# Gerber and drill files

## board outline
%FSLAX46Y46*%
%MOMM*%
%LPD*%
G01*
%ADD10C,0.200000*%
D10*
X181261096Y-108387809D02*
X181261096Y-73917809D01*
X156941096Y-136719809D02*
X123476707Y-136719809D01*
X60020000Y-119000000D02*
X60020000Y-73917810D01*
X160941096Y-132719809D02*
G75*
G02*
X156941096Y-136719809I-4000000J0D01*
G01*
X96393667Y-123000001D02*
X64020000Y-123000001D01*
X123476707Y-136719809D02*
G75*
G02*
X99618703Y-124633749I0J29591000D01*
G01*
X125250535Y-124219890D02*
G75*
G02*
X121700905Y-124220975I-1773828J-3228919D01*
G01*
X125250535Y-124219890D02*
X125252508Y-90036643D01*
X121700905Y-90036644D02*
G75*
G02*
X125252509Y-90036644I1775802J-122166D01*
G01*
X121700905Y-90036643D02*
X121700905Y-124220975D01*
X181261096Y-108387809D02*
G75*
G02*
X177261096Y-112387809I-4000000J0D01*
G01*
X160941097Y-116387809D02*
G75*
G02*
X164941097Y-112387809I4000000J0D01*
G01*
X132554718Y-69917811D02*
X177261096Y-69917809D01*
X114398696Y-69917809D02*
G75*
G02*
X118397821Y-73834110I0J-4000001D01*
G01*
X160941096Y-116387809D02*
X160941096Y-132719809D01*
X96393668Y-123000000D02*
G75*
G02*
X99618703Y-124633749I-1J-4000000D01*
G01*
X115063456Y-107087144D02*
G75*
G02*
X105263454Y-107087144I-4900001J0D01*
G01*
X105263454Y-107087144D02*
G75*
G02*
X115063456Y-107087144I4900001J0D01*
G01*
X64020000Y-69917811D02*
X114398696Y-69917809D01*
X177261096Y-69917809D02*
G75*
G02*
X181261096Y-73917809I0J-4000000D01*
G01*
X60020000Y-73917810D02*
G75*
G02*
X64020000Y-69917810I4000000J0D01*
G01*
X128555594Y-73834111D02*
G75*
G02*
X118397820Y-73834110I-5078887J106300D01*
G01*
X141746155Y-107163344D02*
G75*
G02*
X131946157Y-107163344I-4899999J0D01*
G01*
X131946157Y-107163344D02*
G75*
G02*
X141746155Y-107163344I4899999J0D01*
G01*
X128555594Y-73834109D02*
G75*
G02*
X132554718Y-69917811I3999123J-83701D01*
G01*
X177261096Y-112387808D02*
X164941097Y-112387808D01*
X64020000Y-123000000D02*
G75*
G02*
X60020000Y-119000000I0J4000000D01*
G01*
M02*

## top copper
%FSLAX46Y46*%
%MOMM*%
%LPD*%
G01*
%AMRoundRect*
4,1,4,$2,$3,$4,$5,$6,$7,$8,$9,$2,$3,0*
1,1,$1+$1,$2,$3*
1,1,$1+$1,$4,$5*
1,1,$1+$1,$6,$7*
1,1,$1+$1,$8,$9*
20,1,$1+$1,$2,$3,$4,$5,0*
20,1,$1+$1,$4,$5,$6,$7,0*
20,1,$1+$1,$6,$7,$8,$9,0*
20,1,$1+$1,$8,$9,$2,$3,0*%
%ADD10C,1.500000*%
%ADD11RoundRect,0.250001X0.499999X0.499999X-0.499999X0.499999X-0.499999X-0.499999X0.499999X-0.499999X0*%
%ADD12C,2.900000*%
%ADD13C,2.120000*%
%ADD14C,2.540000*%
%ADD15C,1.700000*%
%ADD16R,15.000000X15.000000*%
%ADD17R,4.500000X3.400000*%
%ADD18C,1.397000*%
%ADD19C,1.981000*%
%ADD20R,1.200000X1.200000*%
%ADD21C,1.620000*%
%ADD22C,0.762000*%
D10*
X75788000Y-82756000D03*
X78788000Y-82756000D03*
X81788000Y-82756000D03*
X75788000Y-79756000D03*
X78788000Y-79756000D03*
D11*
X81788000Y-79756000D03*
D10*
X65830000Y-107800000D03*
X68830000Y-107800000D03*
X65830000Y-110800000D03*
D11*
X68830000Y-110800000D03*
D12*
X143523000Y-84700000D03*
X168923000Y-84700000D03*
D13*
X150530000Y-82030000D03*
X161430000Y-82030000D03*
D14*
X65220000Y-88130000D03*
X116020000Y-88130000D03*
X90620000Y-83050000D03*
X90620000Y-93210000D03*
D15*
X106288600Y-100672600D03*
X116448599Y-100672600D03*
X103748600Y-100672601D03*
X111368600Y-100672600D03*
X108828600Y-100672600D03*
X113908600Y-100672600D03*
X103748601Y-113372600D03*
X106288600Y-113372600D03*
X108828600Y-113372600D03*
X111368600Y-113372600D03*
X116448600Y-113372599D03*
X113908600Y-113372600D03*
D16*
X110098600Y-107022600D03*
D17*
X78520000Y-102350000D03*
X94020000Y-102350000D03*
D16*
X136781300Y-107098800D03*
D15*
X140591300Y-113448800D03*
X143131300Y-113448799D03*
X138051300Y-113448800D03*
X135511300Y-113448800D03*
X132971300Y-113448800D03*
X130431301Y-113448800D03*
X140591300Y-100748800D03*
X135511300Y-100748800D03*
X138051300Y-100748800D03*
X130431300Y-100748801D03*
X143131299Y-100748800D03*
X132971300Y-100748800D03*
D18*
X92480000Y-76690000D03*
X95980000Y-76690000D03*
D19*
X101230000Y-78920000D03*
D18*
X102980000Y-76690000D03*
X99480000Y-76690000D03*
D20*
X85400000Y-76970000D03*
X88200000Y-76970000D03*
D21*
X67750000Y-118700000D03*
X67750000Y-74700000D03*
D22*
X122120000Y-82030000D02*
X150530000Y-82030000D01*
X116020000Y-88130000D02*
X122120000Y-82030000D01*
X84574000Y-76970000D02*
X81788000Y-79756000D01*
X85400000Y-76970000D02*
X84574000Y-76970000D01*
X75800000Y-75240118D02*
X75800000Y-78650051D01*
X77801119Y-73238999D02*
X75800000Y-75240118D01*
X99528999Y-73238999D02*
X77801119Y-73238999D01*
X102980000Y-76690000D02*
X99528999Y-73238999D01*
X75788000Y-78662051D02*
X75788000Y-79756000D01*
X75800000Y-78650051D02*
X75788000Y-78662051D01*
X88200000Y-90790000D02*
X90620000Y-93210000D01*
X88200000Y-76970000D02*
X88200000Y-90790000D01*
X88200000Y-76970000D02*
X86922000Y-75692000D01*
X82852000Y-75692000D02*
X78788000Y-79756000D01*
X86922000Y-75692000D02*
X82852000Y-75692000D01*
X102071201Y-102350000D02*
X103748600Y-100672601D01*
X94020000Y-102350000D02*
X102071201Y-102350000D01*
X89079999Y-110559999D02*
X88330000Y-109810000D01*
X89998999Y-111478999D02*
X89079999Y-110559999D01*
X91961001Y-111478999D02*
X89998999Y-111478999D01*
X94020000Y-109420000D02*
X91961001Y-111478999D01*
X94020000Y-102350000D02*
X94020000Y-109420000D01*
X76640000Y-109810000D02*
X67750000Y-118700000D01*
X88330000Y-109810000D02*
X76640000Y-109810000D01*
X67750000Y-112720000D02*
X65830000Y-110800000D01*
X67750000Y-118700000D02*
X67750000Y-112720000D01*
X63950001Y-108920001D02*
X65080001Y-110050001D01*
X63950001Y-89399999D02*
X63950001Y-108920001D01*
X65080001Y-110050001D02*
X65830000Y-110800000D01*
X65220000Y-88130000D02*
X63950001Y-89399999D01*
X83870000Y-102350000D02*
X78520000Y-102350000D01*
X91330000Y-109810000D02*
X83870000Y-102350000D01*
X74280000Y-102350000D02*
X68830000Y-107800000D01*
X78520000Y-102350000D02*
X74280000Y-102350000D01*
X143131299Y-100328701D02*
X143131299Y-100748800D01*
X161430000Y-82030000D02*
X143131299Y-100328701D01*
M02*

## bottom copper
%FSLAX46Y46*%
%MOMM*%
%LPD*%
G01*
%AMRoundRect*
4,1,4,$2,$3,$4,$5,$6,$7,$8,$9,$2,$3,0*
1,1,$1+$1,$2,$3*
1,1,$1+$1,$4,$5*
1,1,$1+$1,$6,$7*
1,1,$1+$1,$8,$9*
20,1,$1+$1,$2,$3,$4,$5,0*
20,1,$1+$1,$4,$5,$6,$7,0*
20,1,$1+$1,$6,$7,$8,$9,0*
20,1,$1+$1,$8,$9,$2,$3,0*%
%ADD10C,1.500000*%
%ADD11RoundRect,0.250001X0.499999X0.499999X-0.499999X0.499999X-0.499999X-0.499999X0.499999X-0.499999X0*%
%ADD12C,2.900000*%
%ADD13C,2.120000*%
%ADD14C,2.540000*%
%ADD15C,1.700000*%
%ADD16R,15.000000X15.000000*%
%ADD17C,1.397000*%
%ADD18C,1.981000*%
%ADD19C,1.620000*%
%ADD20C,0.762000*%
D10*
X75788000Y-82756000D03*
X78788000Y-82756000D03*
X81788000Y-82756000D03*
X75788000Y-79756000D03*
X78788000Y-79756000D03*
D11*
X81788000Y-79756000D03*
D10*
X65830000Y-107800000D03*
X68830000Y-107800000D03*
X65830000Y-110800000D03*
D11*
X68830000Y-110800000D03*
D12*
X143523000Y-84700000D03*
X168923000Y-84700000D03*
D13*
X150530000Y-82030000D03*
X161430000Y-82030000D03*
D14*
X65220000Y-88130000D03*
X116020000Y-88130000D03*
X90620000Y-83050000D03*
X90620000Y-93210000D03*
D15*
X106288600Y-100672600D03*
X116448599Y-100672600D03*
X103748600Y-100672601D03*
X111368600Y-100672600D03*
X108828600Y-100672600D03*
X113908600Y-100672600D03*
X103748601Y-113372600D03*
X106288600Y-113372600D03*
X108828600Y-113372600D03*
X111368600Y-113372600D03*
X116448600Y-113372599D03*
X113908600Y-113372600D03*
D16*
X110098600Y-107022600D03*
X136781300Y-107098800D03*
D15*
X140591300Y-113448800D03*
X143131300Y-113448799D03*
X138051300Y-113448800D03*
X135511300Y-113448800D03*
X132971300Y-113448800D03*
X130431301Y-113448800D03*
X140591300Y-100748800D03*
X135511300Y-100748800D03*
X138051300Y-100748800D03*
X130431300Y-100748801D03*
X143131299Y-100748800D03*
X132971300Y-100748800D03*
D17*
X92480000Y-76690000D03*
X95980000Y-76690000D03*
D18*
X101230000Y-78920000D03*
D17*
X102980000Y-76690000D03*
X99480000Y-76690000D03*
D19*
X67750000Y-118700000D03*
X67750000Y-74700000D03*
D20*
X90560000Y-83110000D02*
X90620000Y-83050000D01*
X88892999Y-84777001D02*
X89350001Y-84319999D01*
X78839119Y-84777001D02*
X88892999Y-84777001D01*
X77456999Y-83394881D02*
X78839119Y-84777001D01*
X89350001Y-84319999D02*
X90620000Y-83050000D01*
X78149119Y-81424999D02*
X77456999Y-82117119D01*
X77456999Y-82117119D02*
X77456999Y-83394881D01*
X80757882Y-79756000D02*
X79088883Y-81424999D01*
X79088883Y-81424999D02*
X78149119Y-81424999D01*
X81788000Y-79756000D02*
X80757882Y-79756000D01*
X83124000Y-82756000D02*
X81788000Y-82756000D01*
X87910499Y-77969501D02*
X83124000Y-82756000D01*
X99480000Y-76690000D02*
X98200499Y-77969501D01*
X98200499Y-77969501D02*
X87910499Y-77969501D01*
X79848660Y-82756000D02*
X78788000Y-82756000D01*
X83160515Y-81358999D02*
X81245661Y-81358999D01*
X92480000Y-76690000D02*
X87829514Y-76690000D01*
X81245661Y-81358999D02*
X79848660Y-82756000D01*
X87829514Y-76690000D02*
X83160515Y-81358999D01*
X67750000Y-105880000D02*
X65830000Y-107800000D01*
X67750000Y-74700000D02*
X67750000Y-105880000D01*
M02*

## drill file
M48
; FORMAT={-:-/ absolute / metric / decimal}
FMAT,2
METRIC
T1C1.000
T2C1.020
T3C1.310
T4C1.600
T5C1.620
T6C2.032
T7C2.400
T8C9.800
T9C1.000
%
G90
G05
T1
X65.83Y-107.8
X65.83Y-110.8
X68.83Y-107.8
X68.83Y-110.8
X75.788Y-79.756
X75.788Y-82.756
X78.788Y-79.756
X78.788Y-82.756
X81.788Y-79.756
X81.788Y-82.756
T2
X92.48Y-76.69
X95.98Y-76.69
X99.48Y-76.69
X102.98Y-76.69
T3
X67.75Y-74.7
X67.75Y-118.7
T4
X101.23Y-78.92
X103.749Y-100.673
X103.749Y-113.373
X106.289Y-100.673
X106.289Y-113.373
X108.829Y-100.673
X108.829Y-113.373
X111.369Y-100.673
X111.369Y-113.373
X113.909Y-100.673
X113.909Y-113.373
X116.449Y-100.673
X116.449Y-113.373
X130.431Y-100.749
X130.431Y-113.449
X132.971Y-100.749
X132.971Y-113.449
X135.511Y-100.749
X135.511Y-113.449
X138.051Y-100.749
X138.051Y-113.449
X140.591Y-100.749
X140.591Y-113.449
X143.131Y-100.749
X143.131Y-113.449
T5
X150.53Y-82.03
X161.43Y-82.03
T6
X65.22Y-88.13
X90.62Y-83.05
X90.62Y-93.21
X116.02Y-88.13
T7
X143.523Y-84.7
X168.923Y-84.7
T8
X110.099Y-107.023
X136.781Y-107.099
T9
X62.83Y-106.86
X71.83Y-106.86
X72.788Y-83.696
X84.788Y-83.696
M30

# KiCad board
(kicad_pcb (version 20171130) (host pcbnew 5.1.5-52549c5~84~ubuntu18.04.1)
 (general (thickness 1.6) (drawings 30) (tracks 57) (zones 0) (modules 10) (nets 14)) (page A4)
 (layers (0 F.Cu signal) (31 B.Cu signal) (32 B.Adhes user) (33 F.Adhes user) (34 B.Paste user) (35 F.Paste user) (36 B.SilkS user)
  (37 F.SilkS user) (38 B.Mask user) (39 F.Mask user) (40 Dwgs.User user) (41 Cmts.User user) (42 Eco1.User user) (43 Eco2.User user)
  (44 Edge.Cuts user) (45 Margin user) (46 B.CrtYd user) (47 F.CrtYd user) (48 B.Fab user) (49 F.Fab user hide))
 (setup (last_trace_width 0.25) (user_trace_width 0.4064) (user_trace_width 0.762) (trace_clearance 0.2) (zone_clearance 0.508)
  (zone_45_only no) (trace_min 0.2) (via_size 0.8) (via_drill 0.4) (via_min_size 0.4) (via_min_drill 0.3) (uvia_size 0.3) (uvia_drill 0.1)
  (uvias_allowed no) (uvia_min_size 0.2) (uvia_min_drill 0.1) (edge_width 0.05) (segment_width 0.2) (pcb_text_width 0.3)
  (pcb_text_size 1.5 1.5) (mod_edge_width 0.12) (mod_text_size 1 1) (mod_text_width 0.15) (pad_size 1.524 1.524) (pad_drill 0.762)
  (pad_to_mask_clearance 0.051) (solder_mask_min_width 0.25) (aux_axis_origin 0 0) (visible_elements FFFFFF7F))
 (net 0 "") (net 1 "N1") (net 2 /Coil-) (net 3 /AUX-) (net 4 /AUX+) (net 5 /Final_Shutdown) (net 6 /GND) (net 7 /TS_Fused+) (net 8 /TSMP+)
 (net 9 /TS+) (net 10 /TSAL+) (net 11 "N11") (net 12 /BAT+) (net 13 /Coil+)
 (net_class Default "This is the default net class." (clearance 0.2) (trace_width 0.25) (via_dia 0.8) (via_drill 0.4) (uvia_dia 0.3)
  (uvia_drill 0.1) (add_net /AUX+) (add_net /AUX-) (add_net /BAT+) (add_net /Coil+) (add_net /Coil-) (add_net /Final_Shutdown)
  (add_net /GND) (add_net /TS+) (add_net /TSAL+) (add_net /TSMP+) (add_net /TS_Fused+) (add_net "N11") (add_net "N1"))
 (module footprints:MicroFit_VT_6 (layer B.Cu) (at 81.788 79.756 180)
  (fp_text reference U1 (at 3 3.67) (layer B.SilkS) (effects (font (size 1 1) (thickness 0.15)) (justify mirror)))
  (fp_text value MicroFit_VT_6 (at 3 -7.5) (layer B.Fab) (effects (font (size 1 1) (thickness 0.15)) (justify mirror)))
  (pad 6 thru_hole circle (at 6 -3 180) (size 1.5 1.5) (drill 1) (layers *.Cu *.Mask) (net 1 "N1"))
  (pad 5 thru_hole circle (at 3 -3 180) (size 1.5 1.5) (drill 1) (layers *.Cu *.Mask) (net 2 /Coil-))
  (pad 4 thru_hole circle (at 0 -3 180) (size 1.5 1.5) (drill 1) (layers *.Cu *.Mask) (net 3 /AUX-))
  (pad 3 thru_hole circle (at 6 0 180) (size 1.5 1.5) (drill 1) (layers *.Cu *.Mask) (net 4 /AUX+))
  (pad 2 thru_hole circle (at 3 0 180) (size 1.5 1.5) (drill 1) (layers *.Cu *.Mask) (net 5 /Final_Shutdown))
  (pad 1 thru_hole roundrect (at 0 0 180) (size 1.5 1.5) (drill 1) (layers *.Cu *.Mask) (roundrect_rratio 0.166667) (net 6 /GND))
  (pad "" np_thru_hole circle (at 9 -3.94 180) (size 1 1) (drill 1) (layers *.Cu *.Mask))
  (pad "" np_thru_hole circle (at -3 -3.94 180) (size 1 1) (drill 1) (layers *.Cu *.Mask)))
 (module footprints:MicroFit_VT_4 (layer F.Cu) (at 68.83 110.8 180)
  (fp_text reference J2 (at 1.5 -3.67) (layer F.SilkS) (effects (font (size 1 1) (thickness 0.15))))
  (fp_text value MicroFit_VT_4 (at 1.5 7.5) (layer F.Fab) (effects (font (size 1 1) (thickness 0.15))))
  (pad 4 thru_hole circle (at 3 3 180) (size 1.5 1.5) (drill 1) (layers *.Cu *.Mask) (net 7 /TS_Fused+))
  (pad 3 thru_hole circle (at 0 3 180) (size 1.5 1.5) (drill 1) (layers *.Cu *.Mask) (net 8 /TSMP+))
  (pad 2 thru_hole circle (at 3 0 180) (size 1.5 1.5) (drill 1) (layers *.Cu *.Mask) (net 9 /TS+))
  (pad 1 thru_hole roundrect (at 0 0 180) (size 1.5 1.5) (drill 1) (layers *.Cu *.Mask) (roundrect_rratio 0.166667) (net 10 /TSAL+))
  (pad "" np_thru_hole circle (at 6 3.94 180) (size 1 1) (drill 1) (layers *.Cu *.Mask))
  (pad "" np_thru_hole circle (at -3 3.94 180) (size 1 1) (drill 1) (layers *.Cu *.Mask)))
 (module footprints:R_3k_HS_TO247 (layer F.Cu) (at 161.43 82.03 180)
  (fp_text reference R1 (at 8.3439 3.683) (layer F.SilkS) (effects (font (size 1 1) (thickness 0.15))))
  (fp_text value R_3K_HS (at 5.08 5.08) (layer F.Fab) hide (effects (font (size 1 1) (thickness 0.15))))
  (pad 5 thru_hole circle (at 17.907 -2.67 180) (size 2.9 2.9) (drill 2.4) (layers *.Cu *.Mask))
  (pad 4 thru_hole circle (at -7.493 -2.67 180) (size 2.9 2.9) (drill 2.4) (layers *.Cu *.Mask))
  (pad 2 thru_hole circle (at 10.9 0 180) (size 2.12 2.12) (drill 1.62) (layers *.Cu *.Mask) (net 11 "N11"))
  (pad 1 thru_hole circle (at 0 0 180) (size 2.12 2.12) (drill 1.62) (layers *.Cu *.Mask) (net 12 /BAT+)))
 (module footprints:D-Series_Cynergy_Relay (layer F.Cu) (at 65.22 88.13)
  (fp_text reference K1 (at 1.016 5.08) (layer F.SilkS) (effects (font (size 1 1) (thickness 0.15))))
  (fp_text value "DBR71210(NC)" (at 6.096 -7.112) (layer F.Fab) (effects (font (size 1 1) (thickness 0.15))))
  (pad 1 thru_hole circle (at 0 0) (size 2.54 2.54) (drill 2.032) (layers *.Cu *.Mask) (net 9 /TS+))
  (pad 2 thru_hole circle (at 50.8 0) (size 2.54 2.54) (drill 2.032) (layers *.Cu *.Mask) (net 11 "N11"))
  (pad 3 thru_hole circle (at 25.4 -5.08) (size 2.54 2.54) (drill 2.032) (layers *.Cu *.Mask) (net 6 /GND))
  (pad 4 thru_hole circle (at 25.4 5.08) (size 2.54 2.54) (drill 2.032) (layers *.Cu *.Mask) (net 5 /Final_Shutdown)))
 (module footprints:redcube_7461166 (layer F.Cu) (at 110.0986 107.0226)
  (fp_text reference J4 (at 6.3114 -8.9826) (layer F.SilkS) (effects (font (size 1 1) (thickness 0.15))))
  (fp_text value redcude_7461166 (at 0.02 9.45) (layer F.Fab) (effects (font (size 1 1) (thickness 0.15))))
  (pad 1 thru_hole circle (at -3.81 -6.35) (size 1.7 1.7) (drill 1.6) (layers *.Cu *.Mask) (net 9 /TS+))
  (pad 1 thru_hole circle (at 6.349999 -6.35) (size 1.7 1.7) (drill 1.6) (layers *.Cu *.Mask) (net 9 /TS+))
  (pad 1 thru_hole circle (at -6.35 -6.349999) (size 1.7 1.7) (drill 1.6) (layers *.Cu *.Mask) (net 9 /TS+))
  (pad 1 thru_hole circle (at 1.27 -6.35) (size 1.7 1.7) (drill 1.6) (layers *.Cu *.Mask) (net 9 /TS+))
  (pad 1 thru_hole circle (at -1.27 -6.35) (size 1.7 1.7) (drill 1.6) (layers *.Cu *.Mask) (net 9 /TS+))
  (pad 1 thru_hole circle (at 3.81 -6.35) (size 1.7 1.7) (drill 1.6) (layers *.Cu *.Mask) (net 9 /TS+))
  (pad 1 thru_hole circle (at -6.349999 6.35) (size 1.7 1.7) (drill 1.6) (layers *.Cu *.Mask) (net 9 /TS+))
  (pad 1 thru_hole circle (at -3.81 6.35) (size 1.7 1.7) (drill 1.6) (layers *.Cu *.Mask) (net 9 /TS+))
  (pad 1 thru_hole circle (at -1.27 6.35) (size 1.7 1.7) (drill 1.6) (layers *.Cu *.Mask) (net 9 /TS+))
  (pad 1 thru_hole circle (at 1.27 6.35) (size 1.7 1.7) (drill 1.6) (layers *.Cu *.Mask) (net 9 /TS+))
  (pad 1 thru_hole circle (at 6.35 6.349999) (size 1.7 1.7) (drill 1.6) (layers *.Cu *.Mask) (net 9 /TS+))
  (pad 1 thru_hole circle (at 3.81 6.35) (size 1.7 1.7) (drill 1.6) (layers *.Cu *.Mask) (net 9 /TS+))
  (pad 1 thru_hole rect (at 0 0) (size 15 15) (drill 9.8) (layers *.Cu *.Mask) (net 9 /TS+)))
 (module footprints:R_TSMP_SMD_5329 (layer F.Cu) (at 86.14 102.35)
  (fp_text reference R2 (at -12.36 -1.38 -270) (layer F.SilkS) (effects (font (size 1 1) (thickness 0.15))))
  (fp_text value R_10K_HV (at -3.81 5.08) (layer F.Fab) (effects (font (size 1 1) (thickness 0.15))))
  (pad 1 smd rect (at -7.62 0) (size 4.5 3.4) (layers F.Cu F.Paste F.Mask) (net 8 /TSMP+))
  (pad 2 smd rect (at 7.88 0) (size 4.5 3.4) (layers F.Cu F.Paste F.Mask) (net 9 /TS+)))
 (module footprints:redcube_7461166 (layer F.Cu) (at 136.7813 107.0988)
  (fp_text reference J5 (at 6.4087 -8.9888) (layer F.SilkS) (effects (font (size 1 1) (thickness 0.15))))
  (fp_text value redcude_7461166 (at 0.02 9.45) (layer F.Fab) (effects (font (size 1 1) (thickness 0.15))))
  (pad 1 thru_hole rect (at 0 0) (size 15 15) (drill 9.8) (layers *.Cu *.Mask) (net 12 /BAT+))
  (pad 1 thru_hole circle (at 3.81 6.35) (size 1.7 1.7) (drill 1.6) (layers *.Cu *.Mask) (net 12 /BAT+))
  (pad 1 thru_hole circle (at 6.35 6.349999) (size 1.7 1.7) (drill 1.6) (layers *.Cu *.Mask) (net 12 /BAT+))
  (pad 1 thru_hole circle (at 1.27 6.35) (size 1.7 1.7) (drill 1.6) (layers *.Cu *.Mask) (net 12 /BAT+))
  (pad 1 thru_hole circle (at -1.27 6.35) (size 1.7 1.7) (drill 1.6) (layers *.Cu *.Mask) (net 12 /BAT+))
  (pad 1 thru_hole circle (at -3.81 6.35) (size 1.7 1.7) (drill 1.6) (layers *.Cu *.Mask) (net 12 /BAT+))
  (pad 1 thru_hole circle (at -6.349999 6.35) (size 1.7 1.7) (drill 1.6) (layers *.Cu *.Mask) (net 12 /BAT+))
  (pad 1 thru_hole circle (at 3.81 -6.35) (size 1.7 1.7) (drill 1.6) (layers *.Cu *.Mask) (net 12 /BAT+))
  (pad 1 thru_hole circle (at -1.27 -6.35) (size 1.7 1.7) (drill 1.6) (layers *.Cu *.Mask) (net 12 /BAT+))
  (pad 1 thru_hole circle (at 1.27 -6.35) (size 1.7 1.7) (drill 1.6) (layers *.Cu *.Mask) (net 12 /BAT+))
  (pad 1 thru_hole circle (at -6.35 -6.349999) (size 1.7 1.7) (drill 1.6) (layers *.Cu *.Mask) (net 12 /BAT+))
  (pad 1 thru_hole circle (at 6.349999 -6.35) (size 1.7 1.7) (drill 1.6) (layers *.Cu *.Mask) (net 12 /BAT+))
  (pad 1 thru_hole circle (at -3.81 -6.35) (size 1.7 1.7) (drill 1.6) (layers *.Cu *.Mask) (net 12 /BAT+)))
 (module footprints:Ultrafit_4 (layer B.Cu) (at 97.73 76.69 270)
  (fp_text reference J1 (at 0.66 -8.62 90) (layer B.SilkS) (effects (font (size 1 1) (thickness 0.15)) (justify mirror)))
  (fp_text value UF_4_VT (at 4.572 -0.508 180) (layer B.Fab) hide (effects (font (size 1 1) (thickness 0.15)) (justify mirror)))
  (pad 4 thru_hole circle (at 0 5.25 90) (size 1.397 1.397) (drill 1.02) (layers *.Cu *.Mask) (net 2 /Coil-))
  (pad 3 thru_hole circle (at 0 1.75 90) (size 1.397 1.397) (drill 1.02) (layers *.Cu *.Mask) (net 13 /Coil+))
  (pad "" thru_hole circle (at 2.23 -3.5 270) (size 1.981 1.981) (drill 1.6) (layers *.Cu *.Mask))
  (pad 1 thru_hole circle (at 0 -5.25 270) (size 1.397 1.397) (drill 1.02) (layers *.Cu *.Mask) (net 4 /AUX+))
  (pad 2 thru_hole circle (at 0 -1.75 270) (size 1.397 1.397) (drill 1.02) (layers *.Cu *.Mask) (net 3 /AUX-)))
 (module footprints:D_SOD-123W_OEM (layer F.Cu) (at 86.8 76.97 180)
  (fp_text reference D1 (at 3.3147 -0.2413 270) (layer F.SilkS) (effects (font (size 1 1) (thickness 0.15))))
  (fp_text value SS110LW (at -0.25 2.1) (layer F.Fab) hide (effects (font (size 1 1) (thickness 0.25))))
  (pad 2 smd rect (at 1.4 0 180) (size 1.2 1.2) (layers F.Cu F.Paste F.Mask) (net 6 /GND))
  (pad 1 smd rect (at -1.4 0 180) (size 1.2 1.2) (layers F.Cu F.Paste F.Mask) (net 5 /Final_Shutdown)))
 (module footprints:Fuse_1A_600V (layer B.Cu) (at 67.75 118.7 90)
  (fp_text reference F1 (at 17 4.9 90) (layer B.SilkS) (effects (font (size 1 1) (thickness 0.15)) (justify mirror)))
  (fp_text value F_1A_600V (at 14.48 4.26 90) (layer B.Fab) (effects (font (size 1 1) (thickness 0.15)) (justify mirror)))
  (pad 1 thru_hole circle (at 0 0 90) (size 1.62 1.62) (drill 1.31) (layers *.Cu *.Mask) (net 9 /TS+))
  (pad 2 thru_hole circle (at 44 0 90) (size 1.62 1.62) (drill 1.31) (layers *.Cu *.Mask) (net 7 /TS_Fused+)))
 (gr_line (start 181.261096 108.387809) (end 181.261096 73.917809) (layer Edge.Cuts) (width 0.2))
 (gr_line (start 156.941096 136.719809) (end 123.476707 136.719809) (layer Edge.Cuts) (width 0.2))
 (gr_line (start 60.02 119) (end 60.02 73.91781) (layer Edge.Cuts) (width 0.2))
 (gr_arc (start 156.941096 132.719809) (end 156.941096 136.719809) (angle -90) (layer Edge.Cuts) (width 0.2))
 (gr_line (start 96.393667 123.000001) (end 64.02 123.000001) (layer Edge.Cuts) (width 0.2))
 (gr_arc (start 123.476707 107.128809) (end 99.618703 124.633749) (angle -53.73199979) (layer Edge.Cuts) (width 0.2))
 (gr_arc (start 123.476707 127.448809) (end 121.700905 124.220975) (angle -302.4) (layer Edge.Cuts) (width 0.2))
 (gr_line (start 125.250535 124.21989) (end 125.252508 90.036643) (layer Edge.Cuts) (width 0.2))
 (gr_arc (start 123.476707 90.15881) (end 125.252509 90.036644) (angle -172.1290943) (layer Edge.Cuts) (width 0.2))
 (gr_line (start 121.700905 90.036643) (end 121.700905 124.220975) (layer Edge.Cuts) (width 0.2))
 (gr_arc (start 177.261096 108.387809) (end 177.261096 112.387809) (angle -90) (layer Edge.Cuts) (width 0.2))
 (gr_arc (start 164.941097 116.387809) (end 164.941097 112.387809) (angle -90) (layer Edge.Cuts) (width 0.2))
 (gr_line (start 132.554718 69.917811) (end 177.261096 69.917809) (layer Edge.Cuts) (width 0.2))
 (gr_arc (start 114.398696 73.91781) (end 118.397821 73.83411) (angle -88.80099199) (layer Edge.Cuts) (width 0.2))
 (gr_line (start 160.941096 116.387809) (end 160.941096 132.719809) (layer Edge.Cuts) (width 0.2))
 (gr_arc (start 96.393667 127) (end 99.618703 124.633749) (angle -53.73200771) (layer Edge.Cuts) (width 0.2))
 (gr_circle (center 110.163455 107.087144) (end 115.063456 107.087144) (layer Edge.Cuts) (width 0.2))
 (gr_line (start 64.02 69.917811) (end 114.398696 69.917809) (layer Edge.Cuts) (width 0.2))
 (gr_arc (start 177.261096 73.917809) (end 181.261096 73.917809) (angle -90.00000194) (layer Edge.Cuts) (width 0.2))
 (gr_arc (start 64.02 73.91781) (end 64.02 69.91781) (angle -90) (layer Edge.Cuts) (width 0.2))
 (gr_arc (start 123.476707 73.727811) (end 118.39782 73.83411) (angle -177.6019899) (layer Edge.Cuts) (width 0.2))
 (gr_circle (center 136.846156 107.163344) (end 141.746155 107.163344) (layer Edge.Cuts) (width 0.2))
 (gr_arc (start 132.554717 73.91781) (end 132.554718 69.917811) (angle -88.80099199) (layer Edge.Cuts) (width 0.2))
 (gr_line (start 177.261096 112.387808) (end 164.941097 112.387808) (layer Edge.Cuts) (width 0.2))
 (gr_arc (start 64.02 119) (end 60.02 119) (angle -90) (layer Edge.Cuts) (width 0.2))
 (segment (start 122.12 82.03) (end 150.53 82.03) (width 0.762) (layer F.Cu) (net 11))
 (segment (start 116.02 88.13) (end 122.12 82.03) (width 0.762) (layer F.Cu) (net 11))
 (segment (start 90.56 83.11) (end 90.62 83.05) (width 0.762) (layer B.Cu) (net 6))
 (segment (start 84.574 76.97) (end 81.788 79.756) (width 0.762) (layer F.Cu) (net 6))
 (segment (start 85.4 76.97) (end 84.574 76.97) (width 0.762) (layer F.Cu) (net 6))
 (segment (start 88.892999 84.777001) (end 89.350001 84.319999) (width 0.762) (layer B.Cu) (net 6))
 (segment (start 78.839119 84.777001) (end 88.892999 84.777001) (width 0.762) (layer B.Cu) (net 6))
 (segment (start 77.456999 83.394881) (end 78.839119 84.777001) (width 0.762) (layer B.Cu) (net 6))
 (segment (start 89.350001 84.319999) (end 90.62 83.05) (width 0.762) (layer B.Cu) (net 6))
 (segment (start 78.149119 81.424999) (end 77.456999 82.117119) (width 0.762) (layer B.Cu) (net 6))
 (segment (start 77.456999 82.117119) (end 77.456999 83.394881) (width 0.762) (layer B.Cu) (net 6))
 (segment (start 80.757882 79.756) (end 79.088883 81.424999) (width 0.762) (layer B.Cu) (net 6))
 (segment (start 79.088883 81.424999) (end 78.149119 81.424999) (width 0.762) (layer B.Cu) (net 6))
 (segment (start 81.788 79.756) (end 80.757882 79.756) (width 0.762) (layer B.Cu) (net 6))
 (segment (start 83.124 82.756) (end 81.788 82.756) (width 0.762) (layer B.Cu) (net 3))
 (segment (start 87.910499 77.969501) (end 83.124 82.756) (width 0.762) (layer B.Cu) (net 3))
 (segment (start 99.48 76.69) (end 98.200499 77.969501) (width 0.762) (layer B.Cu) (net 3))
 (segment (start 98.200499 77.969501) (end 87.910499 77.969501) (width 0.762) (layer B.Cu) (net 3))
 (segment (start 79.84866 82.756) (end 78.788 82.756) (width 0.762) (layer B.Cu) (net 2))
 (segment (start 83.160515 81.358999) (end 81.245661 81.358999) (width 0.762) (layer B.Cu) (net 2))
 (segment (start 92.48 76.69) (end 87.829514 76.69) (width 0.762) (layer B.Cu) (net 2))
 (segment (start 81.245661 81.358999) (end 79.84866 82.756) (width 0.762) (layer B.Cu) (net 2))
 (segment (start 87.829514 76.69) (end 83.160515 81.358999) (width 0.762) (layer B.Cu) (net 2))
 (segment (start 75.8 75.240118) (end 75.8 78.650051) (width 0.762) (layer F.Cu) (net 4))
 (segment (start 77.801119 73.238999) (end 75.8 75.240118) (width 0.762) (layer F.Cu) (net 4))
 (segment (start 99.528999 73.238999) (end 77.801119 73.238999) (width 0.762) (layer F.Cu) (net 4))
 (segment (start 102.98 76.69) (end 99.528999 73.238999) (width 0.762) (layer F.Cu) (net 4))
 (segment (start 75.788 78.662051) (end 75.788 79.756) (width 0.762) (layer F.Cu) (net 4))
 (segment (start 75.8 78.650051) (end 75.788 78.662051) (width 0.762) (layer F.Cu) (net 4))
 (segment (start 88.2 90.79) (end 90.62 93.21) (width 0.762) (layer F.Cu) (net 5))
 (segment (start 88.2 76.97) (end 88.2 90.79) (width 0.762) (layer F.Cu) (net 5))
 (segment (start 88.2 76.97) (end 86.922 75.692) (width 0.762) (layer F.Cu) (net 5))
 (segment (start 82.852 75.692) (end 78.788 79.756) (width 0.762) (layer F.Cu) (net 5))
 (segment (start 86.922 75.692) (end 82.852 75.692) (width 0.762) (layer F.Cu) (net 5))
 (segment (start 102.071201 102.35) (end 103.7486 100.672601) (width 0.762) (layer F.Cu) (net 9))
 (segment (start 94.02 102.35) (end 102.071201 102.35) (width 0.762) (layer F.Cu) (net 9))
 (segment (start 89.079999 110.559999) (end 88.33 109.81) (width 0.762) (layer F.Cu) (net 9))
 (segment (start 89.998999 111.478999) (end 89.079999 110.559999) (width 0.762) (layer F.Cu) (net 9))
 (segment (start 91.961001 111.478999) (end 89.998999 111.478999) (width 0.762) (layer F.Cu) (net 9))
 (segment (start 94.02 109.42) (end 91.961001 111.478999) (width 0.762) (layer F.Cu) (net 9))
 (segment (start 94.02 102.35) (end 94.02 109.42) (width 0.762) (layer F.Cu) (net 9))
 (segment (start 76.64 109.81) (end 67.75 118.7) (width 0.762) (layer F.Cu) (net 9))
 (segment (start 88.33 109.81) (end 76.64 109.81) (width 0.762) (layer F.Cu) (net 9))
 (segment (start 67.75 112.72) (end 65.83 110.8) (width 0.762) (layer F.Cu) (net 9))
 (segment (start 67.75 118.7) (end 67.75 112.72) (width 0.762) (layer F.Cu) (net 9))
 (segment (start 63.950001 108.920001) (end 65.080001 110.050001) (width 0.762) (layer F.Cu) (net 9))
 (segment (start 63.950001 89.399999) (end 63.950001 108.920001) (width 0.762) (layer F.Cu) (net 9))
 (segment (start 65.080001 110.050001) (end 65.83 110.8) (width 0.762) (layer F.Cu) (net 9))
 (segment (start 65.22 88.13) (end 63.950001 89.399999) (width 0.762) (layer F.Cu) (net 9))
 (segment (start 67.75 105.88) (end 65.83 107.8) (width 0.762) (layer B.Cu) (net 7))
 (segment (start 67.75 74.7) (end 67.75 105.88) (width 0.762) (layer B.Cu) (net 7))
 (segment (start 83.87 102.35) (end 78.52 102.35) (width 0.762) (layer F.Cu) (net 8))
 (segment (start 91.33 109.81) (end 83.87 102.35) (width 0.762) (layer F.Cu) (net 8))
 (segment (start 74.28 102.35) (end 68.83 107.8) (width 0.762) (layer F.Cu) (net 8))
 (segment (start 78.52 102.35) (end 74.28 102.35) (width 0.762) (layer F.Cu) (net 8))
 (segment (start 143.131299 100.328701) (end 143.131299 100.7488) (width 0.762) (layer F.Cu) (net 12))
 (segment (start 161.43 82.03) (end 143.131299 100.328701) (width 0.762) (layer F.Cu) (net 12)))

